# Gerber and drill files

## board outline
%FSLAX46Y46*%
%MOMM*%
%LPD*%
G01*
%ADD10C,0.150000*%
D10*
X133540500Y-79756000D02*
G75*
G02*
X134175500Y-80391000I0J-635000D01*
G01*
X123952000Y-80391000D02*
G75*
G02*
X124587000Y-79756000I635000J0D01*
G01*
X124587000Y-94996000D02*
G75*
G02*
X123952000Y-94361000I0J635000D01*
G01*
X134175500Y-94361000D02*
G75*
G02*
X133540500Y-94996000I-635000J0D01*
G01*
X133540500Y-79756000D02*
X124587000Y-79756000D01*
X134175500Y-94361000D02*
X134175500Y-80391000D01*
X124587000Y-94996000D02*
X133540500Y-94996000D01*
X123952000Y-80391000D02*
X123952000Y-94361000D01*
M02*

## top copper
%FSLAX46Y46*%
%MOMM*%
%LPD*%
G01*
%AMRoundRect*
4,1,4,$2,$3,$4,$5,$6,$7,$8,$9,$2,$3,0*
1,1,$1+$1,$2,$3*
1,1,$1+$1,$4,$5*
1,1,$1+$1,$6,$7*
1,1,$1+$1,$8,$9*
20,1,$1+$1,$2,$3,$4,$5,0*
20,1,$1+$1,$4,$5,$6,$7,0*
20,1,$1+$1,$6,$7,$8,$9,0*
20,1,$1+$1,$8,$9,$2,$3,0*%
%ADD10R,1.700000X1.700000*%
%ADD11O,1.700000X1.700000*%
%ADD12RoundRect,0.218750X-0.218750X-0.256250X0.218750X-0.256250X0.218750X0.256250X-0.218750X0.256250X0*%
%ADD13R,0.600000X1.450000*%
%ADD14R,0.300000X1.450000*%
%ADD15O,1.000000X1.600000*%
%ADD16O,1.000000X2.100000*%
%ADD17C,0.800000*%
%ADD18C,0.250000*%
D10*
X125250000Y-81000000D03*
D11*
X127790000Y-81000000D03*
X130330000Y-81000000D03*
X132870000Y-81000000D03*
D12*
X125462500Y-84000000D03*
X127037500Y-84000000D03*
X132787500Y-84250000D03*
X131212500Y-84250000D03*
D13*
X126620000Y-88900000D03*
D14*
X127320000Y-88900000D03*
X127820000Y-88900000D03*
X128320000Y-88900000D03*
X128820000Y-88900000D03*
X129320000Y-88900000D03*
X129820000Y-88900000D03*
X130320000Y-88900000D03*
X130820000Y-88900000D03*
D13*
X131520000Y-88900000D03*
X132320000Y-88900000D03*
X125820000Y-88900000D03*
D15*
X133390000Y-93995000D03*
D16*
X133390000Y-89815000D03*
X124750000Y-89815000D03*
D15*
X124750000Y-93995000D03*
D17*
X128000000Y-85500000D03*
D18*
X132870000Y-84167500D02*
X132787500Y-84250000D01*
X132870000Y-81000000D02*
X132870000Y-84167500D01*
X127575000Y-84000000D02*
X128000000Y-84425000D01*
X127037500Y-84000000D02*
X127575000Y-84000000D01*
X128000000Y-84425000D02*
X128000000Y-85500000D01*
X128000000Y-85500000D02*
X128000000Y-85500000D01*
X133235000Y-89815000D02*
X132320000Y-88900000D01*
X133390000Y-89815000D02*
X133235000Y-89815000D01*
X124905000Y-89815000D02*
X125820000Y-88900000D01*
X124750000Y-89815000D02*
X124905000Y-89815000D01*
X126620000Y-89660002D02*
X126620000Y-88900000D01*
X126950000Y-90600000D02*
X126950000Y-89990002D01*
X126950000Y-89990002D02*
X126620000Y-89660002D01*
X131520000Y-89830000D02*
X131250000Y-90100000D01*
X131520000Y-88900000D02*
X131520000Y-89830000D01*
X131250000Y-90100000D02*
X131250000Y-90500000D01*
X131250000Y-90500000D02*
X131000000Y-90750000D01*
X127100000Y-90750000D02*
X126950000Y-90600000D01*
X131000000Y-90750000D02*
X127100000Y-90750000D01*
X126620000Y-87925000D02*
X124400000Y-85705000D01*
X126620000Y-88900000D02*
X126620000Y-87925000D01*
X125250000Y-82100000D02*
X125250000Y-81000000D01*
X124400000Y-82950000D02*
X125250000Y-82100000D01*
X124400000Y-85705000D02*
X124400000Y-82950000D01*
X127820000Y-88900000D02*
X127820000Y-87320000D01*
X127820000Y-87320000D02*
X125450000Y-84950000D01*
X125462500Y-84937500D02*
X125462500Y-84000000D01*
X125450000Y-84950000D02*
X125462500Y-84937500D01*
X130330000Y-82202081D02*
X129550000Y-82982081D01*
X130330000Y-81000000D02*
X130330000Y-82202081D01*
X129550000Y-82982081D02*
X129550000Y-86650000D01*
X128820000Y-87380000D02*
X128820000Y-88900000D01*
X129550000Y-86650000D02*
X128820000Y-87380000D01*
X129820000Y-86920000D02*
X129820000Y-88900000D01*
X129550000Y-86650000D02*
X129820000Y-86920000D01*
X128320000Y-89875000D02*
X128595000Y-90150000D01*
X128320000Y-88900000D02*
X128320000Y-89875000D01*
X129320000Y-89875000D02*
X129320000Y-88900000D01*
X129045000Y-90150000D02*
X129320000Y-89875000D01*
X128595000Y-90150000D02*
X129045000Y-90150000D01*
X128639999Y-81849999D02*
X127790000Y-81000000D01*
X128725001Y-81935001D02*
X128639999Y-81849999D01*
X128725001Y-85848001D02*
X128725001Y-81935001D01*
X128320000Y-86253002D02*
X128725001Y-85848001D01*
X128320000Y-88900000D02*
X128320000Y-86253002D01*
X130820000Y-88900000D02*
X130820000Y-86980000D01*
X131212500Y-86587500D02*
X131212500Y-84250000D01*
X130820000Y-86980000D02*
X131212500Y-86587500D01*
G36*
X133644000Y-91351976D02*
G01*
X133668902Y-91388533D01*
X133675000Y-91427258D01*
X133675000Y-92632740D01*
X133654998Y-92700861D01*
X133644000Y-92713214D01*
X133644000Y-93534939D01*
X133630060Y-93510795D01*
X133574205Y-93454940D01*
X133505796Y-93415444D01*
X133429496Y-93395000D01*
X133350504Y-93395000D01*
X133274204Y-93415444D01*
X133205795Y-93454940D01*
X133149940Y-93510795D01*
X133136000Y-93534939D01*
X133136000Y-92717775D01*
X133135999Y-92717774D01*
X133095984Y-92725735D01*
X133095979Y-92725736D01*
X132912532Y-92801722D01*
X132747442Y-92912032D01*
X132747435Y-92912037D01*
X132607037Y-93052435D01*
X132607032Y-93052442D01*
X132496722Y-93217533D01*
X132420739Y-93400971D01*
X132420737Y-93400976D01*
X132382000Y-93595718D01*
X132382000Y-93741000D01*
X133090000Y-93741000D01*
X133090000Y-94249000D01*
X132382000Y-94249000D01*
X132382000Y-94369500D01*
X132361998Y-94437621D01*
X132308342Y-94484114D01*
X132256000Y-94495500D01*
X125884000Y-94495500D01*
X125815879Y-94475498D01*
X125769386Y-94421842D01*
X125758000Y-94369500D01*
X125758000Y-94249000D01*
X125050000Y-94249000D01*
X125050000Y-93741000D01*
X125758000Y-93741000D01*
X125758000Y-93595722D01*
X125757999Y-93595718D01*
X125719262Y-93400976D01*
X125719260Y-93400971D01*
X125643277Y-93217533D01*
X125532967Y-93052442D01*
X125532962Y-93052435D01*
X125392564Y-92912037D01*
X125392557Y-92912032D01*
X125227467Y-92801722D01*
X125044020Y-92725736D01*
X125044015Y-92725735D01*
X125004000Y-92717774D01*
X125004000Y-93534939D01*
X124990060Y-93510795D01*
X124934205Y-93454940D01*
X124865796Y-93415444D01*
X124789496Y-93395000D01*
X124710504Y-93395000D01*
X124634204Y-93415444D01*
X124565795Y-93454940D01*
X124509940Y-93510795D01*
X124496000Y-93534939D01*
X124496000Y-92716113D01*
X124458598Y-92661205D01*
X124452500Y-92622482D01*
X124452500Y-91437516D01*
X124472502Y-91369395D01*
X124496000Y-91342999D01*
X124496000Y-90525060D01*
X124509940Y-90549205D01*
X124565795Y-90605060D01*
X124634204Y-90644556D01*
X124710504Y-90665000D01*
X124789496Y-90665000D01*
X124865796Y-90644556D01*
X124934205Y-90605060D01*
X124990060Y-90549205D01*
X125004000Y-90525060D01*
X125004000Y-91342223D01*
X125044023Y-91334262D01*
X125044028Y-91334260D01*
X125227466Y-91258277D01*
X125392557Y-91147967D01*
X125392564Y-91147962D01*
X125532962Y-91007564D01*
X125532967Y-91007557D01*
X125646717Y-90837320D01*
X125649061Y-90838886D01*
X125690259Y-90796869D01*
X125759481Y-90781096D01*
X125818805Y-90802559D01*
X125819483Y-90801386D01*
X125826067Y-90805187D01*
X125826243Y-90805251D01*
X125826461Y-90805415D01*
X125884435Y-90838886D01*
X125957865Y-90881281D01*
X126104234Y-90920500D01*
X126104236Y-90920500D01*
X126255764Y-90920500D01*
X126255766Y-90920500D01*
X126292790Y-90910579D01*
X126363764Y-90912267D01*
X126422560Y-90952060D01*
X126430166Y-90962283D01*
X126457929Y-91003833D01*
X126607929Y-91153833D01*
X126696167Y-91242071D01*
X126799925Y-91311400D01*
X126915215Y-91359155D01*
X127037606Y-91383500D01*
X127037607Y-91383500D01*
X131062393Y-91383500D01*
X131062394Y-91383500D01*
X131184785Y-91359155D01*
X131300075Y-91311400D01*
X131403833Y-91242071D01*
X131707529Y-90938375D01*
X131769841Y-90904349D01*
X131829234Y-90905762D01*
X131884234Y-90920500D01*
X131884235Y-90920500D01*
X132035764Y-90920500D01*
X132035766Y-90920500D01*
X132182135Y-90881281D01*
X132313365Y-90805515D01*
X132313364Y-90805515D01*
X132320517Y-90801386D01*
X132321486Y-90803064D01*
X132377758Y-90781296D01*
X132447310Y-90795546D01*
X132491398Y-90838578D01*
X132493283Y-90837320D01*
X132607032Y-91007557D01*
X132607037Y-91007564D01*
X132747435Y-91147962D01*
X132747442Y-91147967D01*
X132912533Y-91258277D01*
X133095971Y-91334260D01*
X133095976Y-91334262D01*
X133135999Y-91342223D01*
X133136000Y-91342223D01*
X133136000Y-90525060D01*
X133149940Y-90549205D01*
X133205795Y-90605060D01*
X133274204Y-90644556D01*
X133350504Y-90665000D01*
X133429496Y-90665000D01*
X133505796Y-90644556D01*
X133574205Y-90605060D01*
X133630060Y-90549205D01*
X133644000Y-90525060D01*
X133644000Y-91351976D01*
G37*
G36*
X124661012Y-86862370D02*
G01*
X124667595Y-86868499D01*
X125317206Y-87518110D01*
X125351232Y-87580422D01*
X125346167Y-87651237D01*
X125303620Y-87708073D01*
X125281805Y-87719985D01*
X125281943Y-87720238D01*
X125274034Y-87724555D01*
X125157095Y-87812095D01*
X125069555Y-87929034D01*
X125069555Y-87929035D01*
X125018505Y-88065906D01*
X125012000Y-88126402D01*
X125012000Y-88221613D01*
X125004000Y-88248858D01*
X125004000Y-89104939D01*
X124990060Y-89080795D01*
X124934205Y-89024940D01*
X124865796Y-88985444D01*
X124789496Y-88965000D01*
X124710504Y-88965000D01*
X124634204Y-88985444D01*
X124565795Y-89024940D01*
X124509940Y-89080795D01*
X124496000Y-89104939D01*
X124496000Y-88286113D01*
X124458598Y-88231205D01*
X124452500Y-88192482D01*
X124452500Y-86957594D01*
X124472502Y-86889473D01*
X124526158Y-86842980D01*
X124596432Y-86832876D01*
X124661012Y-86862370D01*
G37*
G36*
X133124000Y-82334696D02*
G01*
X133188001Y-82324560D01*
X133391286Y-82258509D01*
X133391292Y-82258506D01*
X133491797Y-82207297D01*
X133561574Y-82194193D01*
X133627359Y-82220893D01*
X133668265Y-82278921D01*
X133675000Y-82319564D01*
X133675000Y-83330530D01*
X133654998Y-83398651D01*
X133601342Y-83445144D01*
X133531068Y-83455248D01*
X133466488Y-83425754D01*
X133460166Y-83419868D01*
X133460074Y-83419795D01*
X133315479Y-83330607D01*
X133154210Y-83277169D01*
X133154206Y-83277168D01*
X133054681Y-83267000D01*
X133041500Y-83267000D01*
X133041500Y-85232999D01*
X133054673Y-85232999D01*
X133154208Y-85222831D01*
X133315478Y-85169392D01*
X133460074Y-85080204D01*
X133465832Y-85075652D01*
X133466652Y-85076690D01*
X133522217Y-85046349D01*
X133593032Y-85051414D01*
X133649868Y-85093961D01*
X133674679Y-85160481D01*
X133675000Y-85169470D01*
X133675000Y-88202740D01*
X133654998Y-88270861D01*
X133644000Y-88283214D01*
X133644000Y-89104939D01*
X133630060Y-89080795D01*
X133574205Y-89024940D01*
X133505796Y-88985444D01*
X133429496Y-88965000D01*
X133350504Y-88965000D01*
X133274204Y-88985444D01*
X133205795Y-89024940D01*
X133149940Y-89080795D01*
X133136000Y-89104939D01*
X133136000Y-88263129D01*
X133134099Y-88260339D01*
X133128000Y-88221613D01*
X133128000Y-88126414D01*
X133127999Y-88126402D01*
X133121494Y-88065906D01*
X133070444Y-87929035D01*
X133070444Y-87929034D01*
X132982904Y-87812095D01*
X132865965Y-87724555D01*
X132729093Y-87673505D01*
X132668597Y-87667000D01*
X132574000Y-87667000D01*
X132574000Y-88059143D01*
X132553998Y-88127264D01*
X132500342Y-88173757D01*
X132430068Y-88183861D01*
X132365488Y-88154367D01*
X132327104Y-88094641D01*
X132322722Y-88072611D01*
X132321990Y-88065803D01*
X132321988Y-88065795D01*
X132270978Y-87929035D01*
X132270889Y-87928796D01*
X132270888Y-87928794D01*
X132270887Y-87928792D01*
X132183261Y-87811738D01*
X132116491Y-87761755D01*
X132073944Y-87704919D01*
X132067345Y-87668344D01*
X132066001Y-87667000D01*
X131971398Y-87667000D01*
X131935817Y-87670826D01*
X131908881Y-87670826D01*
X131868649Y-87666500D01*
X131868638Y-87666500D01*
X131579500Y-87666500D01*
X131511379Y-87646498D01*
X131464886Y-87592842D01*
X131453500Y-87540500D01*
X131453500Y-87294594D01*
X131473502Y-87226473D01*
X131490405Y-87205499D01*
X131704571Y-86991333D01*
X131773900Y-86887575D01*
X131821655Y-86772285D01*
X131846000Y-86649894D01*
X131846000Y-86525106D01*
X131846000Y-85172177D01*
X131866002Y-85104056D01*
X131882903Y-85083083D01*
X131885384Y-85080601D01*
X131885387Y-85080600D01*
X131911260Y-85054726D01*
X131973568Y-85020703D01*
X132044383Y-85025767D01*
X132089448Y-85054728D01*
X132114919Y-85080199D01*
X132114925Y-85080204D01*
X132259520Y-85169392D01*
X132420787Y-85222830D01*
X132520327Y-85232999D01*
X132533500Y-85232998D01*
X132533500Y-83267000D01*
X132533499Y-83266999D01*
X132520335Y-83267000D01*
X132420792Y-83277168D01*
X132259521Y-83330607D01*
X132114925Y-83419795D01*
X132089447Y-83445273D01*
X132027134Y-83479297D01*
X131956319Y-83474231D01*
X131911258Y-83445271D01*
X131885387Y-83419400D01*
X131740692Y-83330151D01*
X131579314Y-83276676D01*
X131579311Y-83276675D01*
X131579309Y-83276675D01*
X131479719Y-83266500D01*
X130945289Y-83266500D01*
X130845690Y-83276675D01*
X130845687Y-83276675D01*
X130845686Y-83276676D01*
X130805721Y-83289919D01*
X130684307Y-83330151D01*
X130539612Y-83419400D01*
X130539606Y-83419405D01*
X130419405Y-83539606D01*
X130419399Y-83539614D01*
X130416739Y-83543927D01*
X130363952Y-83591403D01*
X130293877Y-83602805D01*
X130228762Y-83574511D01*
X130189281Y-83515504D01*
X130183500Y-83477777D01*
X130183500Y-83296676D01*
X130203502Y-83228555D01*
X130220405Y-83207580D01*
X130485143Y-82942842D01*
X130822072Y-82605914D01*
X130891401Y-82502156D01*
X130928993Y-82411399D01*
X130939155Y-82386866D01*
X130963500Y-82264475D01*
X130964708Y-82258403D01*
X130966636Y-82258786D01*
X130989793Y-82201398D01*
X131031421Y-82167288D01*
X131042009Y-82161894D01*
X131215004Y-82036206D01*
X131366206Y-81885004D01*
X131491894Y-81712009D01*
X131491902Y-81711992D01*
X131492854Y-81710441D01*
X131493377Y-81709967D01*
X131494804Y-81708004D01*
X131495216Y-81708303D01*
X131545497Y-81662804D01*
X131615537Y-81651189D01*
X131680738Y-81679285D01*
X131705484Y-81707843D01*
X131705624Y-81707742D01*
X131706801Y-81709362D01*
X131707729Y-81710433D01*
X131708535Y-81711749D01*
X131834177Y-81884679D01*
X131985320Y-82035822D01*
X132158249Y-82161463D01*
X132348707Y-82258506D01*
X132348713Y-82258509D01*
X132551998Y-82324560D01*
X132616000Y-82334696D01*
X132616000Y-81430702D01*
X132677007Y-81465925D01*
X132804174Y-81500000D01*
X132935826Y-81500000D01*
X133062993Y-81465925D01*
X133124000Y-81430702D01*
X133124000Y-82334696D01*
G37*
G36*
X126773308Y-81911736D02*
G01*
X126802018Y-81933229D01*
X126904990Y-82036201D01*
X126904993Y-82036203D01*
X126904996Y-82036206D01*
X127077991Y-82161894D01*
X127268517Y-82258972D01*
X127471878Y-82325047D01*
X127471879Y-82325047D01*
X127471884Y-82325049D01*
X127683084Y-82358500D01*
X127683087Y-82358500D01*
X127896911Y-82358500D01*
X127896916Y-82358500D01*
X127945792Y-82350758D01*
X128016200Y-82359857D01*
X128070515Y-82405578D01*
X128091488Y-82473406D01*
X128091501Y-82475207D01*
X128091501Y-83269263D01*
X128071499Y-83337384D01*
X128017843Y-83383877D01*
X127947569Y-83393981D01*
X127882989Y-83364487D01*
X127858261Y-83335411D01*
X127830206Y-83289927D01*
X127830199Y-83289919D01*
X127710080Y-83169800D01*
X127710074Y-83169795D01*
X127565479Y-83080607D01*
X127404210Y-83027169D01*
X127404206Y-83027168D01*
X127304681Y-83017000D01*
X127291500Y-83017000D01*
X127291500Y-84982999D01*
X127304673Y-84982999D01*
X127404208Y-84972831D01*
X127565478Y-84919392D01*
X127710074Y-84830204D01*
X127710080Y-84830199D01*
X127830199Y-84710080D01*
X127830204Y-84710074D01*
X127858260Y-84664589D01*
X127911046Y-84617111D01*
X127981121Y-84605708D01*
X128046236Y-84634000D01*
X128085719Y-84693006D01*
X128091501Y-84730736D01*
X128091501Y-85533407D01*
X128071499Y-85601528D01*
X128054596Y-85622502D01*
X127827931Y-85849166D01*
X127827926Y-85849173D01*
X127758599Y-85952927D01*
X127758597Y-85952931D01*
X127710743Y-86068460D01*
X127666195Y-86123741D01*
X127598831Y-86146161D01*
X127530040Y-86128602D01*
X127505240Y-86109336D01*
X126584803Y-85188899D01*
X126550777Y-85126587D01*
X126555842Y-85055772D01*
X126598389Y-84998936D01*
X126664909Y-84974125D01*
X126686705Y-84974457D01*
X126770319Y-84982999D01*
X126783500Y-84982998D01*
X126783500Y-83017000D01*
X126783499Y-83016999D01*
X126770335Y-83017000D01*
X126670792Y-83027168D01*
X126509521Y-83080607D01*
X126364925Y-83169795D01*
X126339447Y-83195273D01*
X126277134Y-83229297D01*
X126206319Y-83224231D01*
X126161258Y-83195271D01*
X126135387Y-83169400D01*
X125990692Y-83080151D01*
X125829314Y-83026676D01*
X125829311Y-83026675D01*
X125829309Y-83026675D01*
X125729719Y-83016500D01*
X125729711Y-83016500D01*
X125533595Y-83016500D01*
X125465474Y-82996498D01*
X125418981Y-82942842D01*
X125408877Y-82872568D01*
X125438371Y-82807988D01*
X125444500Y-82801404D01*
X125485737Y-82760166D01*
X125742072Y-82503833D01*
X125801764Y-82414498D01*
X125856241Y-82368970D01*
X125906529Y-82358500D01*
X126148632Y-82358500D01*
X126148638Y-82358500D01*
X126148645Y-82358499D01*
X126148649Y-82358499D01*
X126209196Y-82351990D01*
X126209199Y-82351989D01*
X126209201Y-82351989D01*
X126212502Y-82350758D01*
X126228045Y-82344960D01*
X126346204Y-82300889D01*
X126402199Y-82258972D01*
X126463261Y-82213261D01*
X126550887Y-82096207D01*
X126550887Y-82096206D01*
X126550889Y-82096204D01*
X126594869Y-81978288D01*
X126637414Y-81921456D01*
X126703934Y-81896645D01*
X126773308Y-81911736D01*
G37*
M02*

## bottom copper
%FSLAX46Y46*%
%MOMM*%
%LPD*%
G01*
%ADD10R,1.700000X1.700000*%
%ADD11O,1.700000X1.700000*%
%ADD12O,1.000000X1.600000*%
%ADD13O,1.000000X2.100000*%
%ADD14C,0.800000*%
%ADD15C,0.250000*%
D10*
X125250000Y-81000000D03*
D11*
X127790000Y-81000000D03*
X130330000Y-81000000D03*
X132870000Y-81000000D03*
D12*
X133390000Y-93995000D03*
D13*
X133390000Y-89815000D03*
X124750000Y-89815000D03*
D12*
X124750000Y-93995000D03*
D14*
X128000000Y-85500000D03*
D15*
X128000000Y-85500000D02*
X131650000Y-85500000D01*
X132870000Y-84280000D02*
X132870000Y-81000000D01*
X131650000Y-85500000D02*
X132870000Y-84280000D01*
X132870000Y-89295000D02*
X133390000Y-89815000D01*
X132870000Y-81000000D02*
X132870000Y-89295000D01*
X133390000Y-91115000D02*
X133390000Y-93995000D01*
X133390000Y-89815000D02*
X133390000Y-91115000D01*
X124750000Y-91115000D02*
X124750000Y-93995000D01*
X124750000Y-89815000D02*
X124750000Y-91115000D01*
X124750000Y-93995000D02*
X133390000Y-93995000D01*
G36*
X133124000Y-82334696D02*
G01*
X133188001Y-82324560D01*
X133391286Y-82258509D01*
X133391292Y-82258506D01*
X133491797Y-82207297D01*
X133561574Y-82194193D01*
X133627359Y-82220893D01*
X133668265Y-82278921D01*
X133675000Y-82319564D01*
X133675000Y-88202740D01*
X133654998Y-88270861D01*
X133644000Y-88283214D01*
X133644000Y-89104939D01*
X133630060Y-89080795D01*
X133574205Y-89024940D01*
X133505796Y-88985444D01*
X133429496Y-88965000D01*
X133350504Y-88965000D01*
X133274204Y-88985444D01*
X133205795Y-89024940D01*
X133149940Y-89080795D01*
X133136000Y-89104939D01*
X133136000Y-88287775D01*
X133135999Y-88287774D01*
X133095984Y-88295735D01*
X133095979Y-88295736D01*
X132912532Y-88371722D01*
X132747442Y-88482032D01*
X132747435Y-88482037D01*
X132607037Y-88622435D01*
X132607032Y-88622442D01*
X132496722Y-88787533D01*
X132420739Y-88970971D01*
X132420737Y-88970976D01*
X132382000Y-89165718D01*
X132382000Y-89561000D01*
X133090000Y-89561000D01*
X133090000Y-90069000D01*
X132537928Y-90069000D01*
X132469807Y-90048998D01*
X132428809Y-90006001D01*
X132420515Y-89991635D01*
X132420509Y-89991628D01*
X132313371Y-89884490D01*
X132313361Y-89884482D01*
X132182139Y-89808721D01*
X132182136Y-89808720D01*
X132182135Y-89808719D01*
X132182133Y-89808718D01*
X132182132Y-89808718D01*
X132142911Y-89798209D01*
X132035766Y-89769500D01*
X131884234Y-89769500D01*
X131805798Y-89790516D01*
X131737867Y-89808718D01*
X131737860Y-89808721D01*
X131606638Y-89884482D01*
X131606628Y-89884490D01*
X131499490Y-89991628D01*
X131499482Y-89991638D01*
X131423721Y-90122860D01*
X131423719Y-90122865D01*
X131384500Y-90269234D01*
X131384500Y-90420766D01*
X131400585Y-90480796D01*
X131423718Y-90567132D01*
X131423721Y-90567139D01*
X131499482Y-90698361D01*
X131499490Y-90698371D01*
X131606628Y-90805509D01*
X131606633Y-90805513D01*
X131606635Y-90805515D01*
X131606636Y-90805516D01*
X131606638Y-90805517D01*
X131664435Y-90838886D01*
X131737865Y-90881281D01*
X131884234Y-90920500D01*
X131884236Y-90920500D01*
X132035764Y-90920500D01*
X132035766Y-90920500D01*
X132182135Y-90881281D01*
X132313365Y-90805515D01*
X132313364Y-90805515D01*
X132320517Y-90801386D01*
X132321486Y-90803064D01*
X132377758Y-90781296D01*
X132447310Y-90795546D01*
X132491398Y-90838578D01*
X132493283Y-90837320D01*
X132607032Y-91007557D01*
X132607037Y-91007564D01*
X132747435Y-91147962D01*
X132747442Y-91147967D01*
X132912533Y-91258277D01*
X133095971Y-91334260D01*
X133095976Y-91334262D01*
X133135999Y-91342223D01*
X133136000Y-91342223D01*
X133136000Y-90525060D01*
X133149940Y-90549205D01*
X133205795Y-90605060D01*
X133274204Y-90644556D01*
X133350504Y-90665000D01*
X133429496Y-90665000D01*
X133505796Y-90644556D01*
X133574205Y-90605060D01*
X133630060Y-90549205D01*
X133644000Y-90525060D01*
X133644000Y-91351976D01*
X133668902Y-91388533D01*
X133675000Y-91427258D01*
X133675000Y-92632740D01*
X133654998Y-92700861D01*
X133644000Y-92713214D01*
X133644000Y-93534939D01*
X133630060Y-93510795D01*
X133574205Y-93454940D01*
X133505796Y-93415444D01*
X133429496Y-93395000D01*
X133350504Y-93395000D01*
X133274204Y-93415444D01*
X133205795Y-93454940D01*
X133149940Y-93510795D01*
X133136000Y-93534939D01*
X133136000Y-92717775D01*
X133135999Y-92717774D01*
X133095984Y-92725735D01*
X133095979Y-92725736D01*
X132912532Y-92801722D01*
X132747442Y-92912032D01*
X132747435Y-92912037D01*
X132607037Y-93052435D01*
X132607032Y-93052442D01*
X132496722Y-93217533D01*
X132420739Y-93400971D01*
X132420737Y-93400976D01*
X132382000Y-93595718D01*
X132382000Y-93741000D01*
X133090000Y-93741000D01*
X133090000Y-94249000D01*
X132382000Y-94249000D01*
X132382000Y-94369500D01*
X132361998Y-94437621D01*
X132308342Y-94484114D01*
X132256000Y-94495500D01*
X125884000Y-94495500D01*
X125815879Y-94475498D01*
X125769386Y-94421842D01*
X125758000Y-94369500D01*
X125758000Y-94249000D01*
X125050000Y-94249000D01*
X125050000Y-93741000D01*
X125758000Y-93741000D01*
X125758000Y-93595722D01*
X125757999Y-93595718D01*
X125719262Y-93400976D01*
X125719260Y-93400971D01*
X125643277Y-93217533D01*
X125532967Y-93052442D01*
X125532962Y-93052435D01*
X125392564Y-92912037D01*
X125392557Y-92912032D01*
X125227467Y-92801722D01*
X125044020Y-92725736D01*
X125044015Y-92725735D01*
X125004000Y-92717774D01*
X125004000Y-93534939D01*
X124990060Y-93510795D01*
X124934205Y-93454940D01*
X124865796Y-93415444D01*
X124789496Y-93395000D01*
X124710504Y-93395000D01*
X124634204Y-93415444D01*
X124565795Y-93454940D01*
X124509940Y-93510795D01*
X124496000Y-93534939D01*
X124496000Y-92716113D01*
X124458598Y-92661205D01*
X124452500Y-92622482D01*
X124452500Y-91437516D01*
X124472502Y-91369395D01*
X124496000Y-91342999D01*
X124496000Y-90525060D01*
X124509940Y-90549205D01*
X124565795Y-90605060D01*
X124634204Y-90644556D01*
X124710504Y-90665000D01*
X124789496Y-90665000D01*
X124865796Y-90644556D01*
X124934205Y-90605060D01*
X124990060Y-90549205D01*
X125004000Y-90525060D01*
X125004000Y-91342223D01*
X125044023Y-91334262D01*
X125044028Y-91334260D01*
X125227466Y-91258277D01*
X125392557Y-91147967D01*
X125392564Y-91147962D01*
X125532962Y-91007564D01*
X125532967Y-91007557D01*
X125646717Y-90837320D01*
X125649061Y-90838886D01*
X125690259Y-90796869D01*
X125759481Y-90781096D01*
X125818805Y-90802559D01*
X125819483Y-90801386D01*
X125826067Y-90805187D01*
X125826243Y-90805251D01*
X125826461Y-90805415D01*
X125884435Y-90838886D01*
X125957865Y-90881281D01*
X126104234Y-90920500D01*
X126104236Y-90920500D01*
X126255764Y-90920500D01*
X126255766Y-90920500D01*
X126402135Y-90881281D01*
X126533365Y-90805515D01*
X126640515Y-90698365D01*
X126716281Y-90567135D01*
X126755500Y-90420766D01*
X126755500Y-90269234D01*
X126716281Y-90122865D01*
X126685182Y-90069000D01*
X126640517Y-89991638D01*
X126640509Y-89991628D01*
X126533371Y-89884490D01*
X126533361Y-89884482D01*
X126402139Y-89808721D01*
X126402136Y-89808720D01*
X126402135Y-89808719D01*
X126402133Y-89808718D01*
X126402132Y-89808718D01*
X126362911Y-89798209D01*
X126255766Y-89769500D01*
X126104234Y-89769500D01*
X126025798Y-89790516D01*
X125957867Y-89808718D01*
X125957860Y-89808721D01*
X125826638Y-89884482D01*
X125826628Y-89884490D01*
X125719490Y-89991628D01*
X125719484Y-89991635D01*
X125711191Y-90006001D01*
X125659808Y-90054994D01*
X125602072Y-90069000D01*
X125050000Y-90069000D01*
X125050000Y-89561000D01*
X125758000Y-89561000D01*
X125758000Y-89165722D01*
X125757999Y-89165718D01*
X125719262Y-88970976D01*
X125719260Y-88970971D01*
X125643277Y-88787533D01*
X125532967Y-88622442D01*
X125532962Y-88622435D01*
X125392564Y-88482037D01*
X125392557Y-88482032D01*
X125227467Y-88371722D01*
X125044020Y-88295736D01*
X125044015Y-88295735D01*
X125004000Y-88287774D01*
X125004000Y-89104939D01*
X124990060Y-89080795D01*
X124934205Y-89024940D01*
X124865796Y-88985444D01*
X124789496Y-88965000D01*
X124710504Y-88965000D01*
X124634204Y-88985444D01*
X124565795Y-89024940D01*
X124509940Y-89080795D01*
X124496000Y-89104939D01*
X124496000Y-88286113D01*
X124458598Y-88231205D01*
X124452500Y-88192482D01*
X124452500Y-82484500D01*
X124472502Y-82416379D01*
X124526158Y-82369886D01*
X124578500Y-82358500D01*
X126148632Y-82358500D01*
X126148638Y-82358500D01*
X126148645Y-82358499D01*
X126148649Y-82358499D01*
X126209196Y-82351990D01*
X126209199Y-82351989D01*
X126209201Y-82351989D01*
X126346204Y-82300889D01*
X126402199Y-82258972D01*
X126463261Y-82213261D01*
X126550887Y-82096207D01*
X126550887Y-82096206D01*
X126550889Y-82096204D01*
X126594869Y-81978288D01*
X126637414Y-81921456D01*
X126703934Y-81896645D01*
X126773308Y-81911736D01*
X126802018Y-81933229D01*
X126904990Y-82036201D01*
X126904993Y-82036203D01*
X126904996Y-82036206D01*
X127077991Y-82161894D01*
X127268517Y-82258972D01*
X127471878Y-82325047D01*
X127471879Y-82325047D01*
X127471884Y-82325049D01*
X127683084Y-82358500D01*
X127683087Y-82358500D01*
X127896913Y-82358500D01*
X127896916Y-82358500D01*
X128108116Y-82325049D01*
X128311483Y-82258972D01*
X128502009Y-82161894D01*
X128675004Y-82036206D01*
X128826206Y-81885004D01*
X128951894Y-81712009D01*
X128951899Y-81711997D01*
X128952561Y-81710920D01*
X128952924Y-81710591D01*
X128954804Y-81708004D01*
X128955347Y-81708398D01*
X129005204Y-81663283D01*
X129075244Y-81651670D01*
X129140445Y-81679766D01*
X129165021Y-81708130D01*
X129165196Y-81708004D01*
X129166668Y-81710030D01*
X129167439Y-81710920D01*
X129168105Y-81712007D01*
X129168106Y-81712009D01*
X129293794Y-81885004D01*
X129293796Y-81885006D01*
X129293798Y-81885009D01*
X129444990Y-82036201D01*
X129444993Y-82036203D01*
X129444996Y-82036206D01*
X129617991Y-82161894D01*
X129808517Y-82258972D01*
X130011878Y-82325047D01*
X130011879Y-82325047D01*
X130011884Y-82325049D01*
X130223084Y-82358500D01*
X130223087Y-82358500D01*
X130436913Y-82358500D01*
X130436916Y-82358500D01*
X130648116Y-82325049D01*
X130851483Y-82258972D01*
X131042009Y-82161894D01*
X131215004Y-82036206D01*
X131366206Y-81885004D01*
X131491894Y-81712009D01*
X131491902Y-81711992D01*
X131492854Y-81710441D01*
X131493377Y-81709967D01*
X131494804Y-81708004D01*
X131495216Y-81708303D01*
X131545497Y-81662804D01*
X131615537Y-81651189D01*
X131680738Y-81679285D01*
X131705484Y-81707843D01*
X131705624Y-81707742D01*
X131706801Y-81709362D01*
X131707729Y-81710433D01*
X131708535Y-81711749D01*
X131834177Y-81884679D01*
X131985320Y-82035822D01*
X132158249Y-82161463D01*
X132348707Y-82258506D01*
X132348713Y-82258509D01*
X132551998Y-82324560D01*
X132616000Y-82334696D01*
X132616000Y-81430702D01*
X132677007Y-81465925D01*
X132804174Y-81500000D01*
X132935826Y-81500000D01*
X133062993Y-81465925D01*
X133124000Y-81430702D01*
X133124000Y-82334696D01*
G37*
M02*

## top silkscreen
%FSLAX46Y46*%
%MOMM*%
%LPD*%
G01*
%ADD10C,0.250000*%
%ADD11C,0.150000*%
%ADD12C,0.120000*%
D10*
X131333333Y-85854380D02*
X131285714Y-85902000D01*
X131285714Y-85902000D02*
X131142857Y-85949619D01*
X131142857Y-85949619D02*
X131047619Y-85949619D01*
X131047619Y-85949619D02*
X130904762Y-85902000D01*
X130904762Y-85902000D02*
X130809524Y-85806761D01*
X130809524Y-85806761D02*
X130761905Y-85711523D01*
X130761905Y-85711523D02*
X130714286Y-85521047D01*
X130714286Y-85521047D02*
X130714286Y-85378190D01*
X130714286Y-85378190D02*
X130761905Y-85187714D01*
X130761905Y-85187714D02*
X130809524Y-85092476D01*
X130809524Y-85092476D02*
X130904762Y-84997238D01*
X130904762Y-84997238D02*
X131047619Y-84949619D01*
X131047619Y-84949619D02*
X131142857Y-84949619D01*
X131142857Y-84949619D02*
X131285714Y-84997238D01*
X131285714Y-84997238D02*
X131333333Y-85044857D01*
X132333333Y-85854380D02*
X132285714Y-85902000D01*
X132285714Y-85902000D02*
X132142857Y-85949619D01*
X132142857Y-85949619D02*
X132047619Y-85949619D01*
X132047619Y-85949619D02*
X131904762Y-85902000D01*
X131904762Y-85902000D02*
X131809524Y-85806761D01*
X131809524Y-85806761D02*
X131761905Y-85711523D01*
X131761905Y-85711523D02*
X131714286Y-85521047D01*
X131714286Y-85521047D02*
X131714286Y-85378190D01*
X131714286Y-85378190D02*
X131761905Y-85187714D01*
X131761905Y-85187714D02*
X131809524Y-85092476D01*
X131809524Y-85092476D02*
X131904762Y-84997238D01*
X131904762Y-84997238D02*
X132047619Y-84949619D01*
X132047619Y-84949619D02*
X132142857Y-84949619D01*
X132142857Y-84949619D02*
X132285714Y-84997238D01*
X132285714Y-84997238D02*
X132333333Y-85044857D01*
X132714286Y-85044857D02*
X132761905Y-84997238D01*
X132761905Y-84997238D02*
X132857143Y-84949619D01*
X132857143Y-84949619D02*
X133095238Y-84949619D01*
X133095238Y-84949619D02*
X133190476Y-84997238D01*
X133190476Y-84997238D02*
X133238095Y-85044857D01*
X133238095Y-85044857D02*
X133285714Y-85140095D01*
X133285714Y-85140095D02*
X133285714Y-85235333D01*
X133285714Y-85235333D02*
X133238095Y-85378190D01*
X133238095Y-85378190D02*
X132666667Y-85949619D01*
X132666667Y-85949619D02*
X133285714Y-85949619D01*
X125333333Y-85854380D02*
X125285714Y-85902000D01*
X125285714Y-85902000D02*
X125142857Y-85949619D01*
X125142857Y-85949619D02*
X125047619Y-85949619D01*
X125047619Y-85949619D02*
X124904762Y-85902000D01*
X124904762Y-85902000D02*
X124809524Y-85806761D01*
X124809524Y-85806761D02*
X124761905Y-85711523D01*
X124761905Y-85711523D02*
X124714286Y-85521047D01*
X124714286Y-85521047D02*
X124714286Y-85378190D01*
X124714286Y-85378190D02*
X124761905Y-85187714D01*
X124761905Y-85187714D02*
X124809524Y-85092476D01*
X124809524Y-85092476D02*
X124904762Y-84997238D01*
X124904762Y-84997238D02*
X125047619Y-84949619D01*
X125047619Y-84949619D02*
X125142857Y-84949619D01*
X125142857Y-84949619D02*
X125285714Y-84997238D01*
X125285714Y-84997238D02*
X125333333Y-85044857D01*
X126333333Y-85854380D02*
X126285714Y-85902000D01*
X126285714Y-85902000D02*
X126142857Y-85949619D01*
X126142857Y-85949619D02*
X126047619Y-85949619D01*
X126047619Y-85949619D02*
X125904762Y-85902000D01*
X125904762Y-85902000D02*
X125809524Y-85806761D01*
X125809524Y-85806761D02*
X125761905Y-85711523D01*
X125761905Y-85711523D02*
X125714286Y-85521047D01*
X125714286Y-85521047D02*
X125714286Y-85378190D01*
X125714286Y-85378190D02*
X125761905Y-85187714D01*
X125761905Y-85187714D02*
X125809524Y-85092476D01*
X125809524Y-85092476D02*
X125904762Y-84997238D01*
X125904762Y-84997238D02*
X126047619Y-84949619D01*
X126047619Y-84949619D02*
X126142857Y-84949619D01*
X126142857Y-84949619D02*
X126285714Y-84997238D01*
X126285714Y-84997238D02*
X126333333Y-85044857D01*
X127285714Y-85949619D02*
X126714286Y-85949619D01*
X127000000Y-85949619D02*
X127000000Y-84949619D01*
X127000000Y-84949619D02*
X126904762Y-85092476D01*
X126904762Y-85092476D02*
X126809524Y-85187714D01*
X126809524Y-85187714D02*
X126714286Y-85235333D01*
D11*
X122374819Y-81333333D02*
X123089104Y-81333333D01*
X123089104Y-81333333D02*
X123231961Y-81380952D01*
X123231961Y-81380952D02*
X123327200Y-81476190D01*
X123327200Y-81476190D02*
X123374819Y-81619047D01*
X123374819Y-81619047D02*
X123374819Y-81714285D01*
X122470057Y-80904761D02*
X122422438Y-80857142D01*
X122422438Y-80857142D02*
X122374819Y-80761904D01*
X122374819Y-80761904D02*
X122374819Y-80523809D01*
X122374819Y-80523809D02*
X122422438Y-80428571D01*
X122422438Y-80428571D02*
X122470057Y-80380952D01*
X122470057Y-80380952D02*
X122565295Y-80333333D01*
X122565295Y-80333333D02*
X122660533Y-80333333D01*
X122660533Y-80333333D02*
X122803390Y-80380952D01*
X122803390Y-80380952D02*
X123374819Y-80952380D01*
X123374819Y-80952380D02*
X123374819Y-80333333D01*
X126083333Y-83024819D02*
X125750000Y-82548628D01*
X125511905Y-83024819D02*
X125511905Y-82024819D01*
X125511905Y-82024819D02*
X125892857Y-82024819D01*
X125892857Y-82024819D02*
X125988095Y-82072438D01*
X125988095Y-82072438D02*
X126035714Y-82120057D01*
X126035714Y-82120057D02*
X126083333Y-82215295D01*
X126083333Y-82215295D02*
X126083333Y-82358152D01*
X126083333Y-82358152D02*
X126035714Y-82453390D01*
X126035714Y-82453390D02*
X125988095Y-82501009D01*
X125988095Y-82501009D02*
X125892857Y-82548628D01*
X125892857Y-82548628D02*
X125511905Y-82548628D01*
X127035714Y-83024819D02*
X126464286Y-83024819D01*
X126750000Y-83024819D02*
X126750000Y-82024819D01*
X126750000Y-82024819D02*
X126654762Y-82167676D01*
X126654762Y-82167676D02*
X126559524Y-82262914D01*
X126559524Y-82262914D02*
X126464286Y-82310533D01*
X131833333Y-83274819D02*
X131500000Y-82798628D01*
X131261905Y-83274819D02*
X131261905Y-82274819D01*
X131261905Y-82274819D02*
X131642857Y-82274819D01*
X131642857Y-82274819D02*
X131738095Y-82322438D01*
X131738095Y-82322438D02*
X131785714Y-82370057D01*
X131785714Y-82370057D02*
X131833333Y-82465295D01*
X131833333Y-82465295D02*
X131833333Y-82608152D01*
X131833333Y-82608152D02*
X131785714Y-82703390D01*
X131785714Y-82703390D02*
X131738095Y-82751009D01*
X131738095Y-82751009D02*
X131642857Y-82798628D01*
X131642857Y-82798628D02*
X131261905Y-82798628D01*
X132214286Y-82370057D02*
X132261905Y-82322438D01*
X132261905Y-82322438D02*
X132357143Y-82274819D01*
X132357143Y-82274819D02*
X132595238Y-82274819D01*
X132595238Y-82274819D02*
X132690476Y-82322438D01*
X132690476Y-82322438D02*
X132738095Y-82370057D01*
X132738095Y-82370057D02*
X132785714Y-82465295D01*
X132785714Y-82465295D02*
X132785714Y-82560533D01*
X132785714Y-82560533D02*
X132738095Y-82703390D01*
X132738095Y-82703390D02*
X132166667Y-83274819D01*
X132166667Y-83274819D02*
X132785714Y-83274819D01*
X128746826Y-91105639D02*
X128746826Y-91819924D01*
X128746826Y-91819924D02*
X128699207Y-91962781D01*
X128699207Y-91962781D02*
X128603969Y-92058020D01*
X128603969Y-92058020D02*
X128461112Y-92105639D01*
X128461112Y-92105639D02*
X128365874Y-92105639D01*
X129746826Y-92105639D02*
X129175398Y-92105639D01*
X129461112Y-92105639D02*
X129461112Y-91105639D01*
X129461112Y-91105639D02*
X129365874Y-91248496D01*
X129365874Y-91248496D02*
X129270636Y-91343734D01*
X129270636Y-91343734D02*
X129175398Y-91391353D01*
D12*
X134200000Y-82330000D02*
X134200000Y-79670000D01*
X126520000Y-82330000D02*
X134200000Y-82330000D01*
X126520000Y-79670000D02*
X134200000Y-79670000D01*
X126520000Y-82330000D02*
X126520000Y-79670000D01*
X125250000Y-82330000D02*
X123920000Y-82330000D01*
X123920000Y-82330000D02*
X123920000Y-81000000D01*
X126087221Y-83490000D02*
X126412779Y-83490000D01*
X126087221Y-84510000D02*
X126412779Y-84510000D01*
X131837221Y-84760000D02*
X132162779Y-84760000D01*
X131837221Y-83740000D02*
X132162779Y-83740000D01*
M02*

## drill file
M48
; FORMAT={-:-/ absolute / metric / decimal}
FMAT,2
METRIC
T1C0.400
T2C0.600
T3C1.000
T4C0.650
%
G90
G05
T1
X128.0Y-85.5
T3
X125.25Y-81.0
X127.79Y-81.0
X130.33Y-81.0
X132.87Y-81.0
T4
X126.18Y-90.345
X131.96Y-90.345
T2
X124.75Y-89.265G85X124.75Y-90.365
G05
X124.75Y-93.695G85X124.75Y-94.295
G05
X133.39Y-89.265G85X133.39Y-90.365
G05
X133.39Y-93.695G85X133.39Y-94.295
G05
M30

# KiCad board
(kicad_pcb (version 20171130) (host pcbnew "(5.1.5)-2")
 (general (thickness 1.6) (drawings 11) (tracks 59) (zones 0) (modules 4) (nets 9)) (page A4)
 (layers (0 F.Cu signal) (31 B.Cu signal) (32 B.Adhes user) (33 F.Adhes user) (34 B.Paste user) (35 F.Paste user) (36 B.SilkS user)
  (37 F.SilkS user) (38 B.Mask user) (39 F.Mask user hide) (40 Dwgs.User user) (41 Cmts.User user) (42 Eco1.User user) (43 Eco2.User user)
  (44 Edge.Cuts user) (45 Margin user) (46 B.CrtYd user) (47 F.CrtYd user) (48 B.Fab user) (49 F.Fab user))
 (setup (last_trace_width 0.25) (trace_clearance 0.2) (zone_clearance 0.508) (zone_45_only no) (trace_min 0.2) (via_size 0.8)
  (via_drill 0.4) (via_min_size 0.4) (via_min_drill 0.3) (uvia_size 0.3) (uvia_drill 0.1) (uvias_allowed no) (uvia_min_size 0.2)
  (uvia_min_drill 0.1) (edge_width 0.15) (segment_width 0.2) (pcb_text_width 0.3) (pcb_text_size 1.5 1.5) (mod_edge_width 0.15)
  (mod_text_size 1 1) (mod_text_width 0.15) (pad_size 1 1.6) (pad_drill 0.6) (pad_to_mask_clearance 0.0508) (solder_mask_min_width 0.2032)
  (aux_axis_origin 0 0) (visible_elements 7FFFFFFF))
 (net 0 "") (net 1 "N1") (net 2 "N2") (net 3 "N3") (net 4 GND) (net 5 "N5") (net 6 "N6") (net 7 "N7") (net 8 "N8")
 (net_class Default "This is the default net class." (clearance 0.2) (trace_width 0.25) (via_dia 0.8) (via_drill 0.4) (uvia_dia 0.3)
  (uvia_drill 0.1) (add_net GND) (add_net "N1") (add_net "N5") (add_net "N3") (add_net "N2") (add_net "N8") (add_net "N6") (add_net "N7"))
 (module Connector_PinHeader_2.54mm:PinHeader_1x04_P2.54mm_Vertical (layer F.Cu) (at 125.25 81 90)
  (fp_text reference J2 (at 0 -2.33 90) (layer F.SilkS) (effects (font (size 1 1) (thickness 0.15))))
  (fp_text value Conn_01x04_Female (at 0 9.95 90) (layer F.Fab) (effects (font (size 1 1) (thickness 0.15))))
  (fp_line (start -1.33 8.95) (end 1.33 8.95) (layer F.SilkS) (width 0.12))
  (fp_line (start -1.33 1.27) (end -1.33 8.95) (layer F.SilkS) (width 0.12))
  (fp_line (start 1.33 1.27) (end 1.33 8.95) (layer F.SilkS) (width 0.12))
  (fp_line (start -1.33 1.27) (end 1.33 1.27) (layer F.SilkS) (width 0.12))
  (fp_line (start -1.33 0) (end -1.33 -1.33) (layer F.SilkS) (width 0.12))
  (fp_line (start -1.33 -1.33) (end 0 -1.33) (layer F.SilkS) (width 0.12))
  (pad 1 thru_hole rect (at 0 0 90) (size 1.7 1.7) (drill 1) (layers *.Cu *.Mask) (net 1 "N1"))
  (pad 2 thru_hole oval (at 0 2.54 90) (size 1.7 1.7) (drill 1) (layers *.Cu *.Mask) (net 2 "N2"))
  (pad 3 thru_hole oval (at 0 5.08 90) (size 1.7 1.7) (drill 1) (layers *.Cu *.Mask) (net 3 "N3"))
  (pad 4 thru_hole oval (at 0 7.62 90) (size 1.7 1.7) (drill 1) (layers *.Cu *.Mask) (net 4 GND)))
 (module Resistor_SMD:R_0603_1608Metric (layer F.Cu) (at 126.25 84)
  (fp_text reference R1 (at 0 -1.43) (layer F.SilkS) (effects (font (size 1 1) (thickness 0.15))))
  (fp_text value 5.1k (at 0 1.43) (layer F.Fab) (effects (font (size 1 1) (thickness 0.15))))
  (fp_line (start -0.162779 -0.51) (end 0.162779 -0.51) (layer F.SilkS) (width 0.12))
  (fp_line (start -0.162779 0.51) (end 0.162779 0.51) (layer F.SilkS) (width 0.12))
  (pad 1 smd roundrect (at -0.7875 0) (size 0.875 0.95) (layers F.Cu F.Paste F.Mask) (roundrect_rratio 0.25) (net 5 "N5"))
  (pad 2 smd roundrect (at 0.7875 0) (size 0.875 0.95) (layers F.Cu F.Paste F.Mask) (roundrect_rratio 0.25) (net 4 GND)))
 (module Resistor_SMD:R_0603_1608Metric (layer F.Cu) (at 132 84.25)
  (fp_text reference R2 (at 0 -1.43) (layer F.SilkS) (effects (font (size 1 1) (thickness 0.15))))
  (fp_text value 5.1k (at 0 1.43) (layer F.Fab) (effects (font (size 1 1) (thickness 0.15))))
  (fp_line (start -0.162779 0.51) (end 0.162779 0.51) (layer F.SilkS) (width 0.12))
  (fp_line (start -0.162779 -0.51) (end 0.162779 -0.51) (layer F.SilkS) (width 0.12))
  (pad 2 smd roundrect (at 0.7875 0) (size 0.875 0.95) (layers F.Cu F.Paste F.Mask) (roundrect_rratio 0.25) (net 4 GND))
  (pad 1 smd roundrect (at -0.7875 0) (size 0.875 0.95) (layers F.Cu F.Paste F.Mask) (roundrect_rratio 0.25) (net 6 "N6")))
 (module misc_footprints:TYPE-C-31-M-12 (layer F.Cu) (at 129.07 88.9)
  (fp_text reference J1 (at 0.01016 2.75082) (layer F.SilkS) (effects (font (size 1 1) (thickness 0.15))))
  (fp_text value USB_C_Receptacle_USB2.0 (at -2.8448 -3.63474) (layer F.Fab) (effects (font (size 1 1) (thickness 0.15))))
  (pad A4|B9 smd rect (at -2.45 0) (size 0.6 1.45) (layers F.Cu F.Paste F.Mask) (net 1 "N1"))
  (pad B8 smd rect (at -1.75 0) (size 0.3 1.45) (layers F.Cu F.Paste F.Mask) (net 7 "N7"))
  (pad A5 smd rect (at -1.25 0) (size 0.3 1.45) (layers F.Cu F.Paste F.Mask) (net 5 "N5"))
  (pad B7 smd rect (at -0.75 0) (size 0.3 1.45) (layers F.Cu F.Paste F.Mask) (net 2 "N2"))
  (pad A6 smd rect (at -0.25 0) (size 0.3 1.45) (layers F.Cu F.Paste F.Mask) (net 3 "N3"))
  (pad A7 smd rect (at 0.25 0) (size 0.3 1.45) (layers F.Cu F.Paste F.Mask) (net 2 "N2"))
  (pad B6 smd rect (at 0.75 0) (size 0.3 1.45) (layers F.Cu F.Paste F.Mask) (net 3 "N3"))
  (pad A8 smd rect (at 1.25 0) (size 0.3 1.45) (layers F.Cu F.Paste F.Mask) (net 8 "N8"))
  (pad B5 smd rect (at 1.75 0) (size 0.3 1.45) (layers F.Cu F.Paste F.Mask) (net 6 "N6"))
  (pad B4|A9 smd rect (at 2.45 0) (size 0.6 1.45) (layers F.Cu F.Paste F.Mask) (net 1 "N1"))
  (pad B1|A12 smd rect (at 3.25 0) (size 0.6 1.45) (layers F.Cu F.Paste F.Mask) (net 4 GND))
  (pad A1|B12 smd rect (at -3.25 0) (size 0.6 1.45) (layers F.Cu F.Paste F.Mask) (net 4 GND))
  (pad GND thru_hole oval (at 4.32 5.095) (size 1 1.6) (drill oval 0.6 1.2) (layers *.Cu *.Mask) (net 4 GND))
  (pad GND thru_hole oval (at 4.32 0.915) (size 1 2.1) (drill oval 0.6 1.7) (layers *.Cu *.Mask) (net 4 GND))
  (pad GND thru_hole oval (at -4.32 0.915) (size 1 2.1) (drill oval 0.6 1.7) (layers *.Cu *.Mask) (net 4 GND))
  (pad GND thru_hole oval (at -4.32 5.095) (size 1 1.6) (drill oval 0.6 1.2) (layers *.Cu *.Mask) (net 4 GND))
  (pad "" np_thru_hole circle (at 2.89 1.445) (size 0.65 0.65) (drill 0.65) (layers *.Cu *.Mask))
  (pad "" np_thru_hole circle (at -2.89 1.445) (size 0.65 0.65) (drill 0.65) (layers *.Cu *.Mask)))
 (gr_arc (start 133.5405 80.391) (end 134.1755 80.391) (angle -90) (layer Edge.Cuts) (width 0.15))
 (gr_arc (start 124.587 80.391) (end 124.587 79.756) (angle -90) (layer Edge.Cuts) (width 0.15))
 (gr_arc (start 124.587 94.361) (end 123.952 94.361) (angle -90) (layer Edge.Cuts) (width 0.15))
 (gr_arc (start 133.5405 94.361) (end 133.5405 94.996) (angle -90) (layer Edge.Cuts) (width 0.15))
 (gr_line (start 133.5405 79.756) (end 124.587 79.756) (layer Edge.Cuts) (width 0.15))
 (gr_line (start 134.1755 94.361) (end 134.1755 80.391) (layer Edge.Cuts) (width 0.15))
 (gr_line (start 124.587 94.996) (end 133.5405 94.996) (layer Edge.Cuts) (width 0.15))
 (gr_line (start 123.952 80.391) (end 123.952 94.361) (layer Edge.Cuts) (width 0.15))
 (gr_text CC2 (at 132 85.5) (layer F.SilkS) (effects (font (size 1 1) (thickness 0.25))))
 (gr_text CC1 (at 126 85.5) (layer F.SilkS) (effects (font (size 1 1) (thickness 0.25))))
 (segment (start 132.87 84.1675) (end 132.7875 84.25) (width 0.25) (layer F.Cu) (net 4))
 (segment (start 132.87 81) (end 132.87 84.1675) (width 0.25) (layer F.Cu) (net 4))
 (segment (start 127.575 84) (end 128 84.425) (width 0.25) (layer F.Cu) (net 4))
 (segment (start 127.0375 84) (end 127.575 84) (width 0.25) (layer F.Cu) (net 4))
 (segment (start 128 84.425) (end 128 85.5) (width 0.25) (layer F.Cu) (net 4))
 (segment (start 128 85.5) (end 128 85.5) (width 0.25) (layer F.Cu) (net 4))
 (via (at 128 85.5) (size 0.8) (drill 0.4) (layers F.Cu B.Cu) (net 4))
 (segment (start 128 85.5) (end 131.65 85.5) (width 0.25) (layer B.Cu) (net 4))
 (segment (start 132.87 84.28) (end 132.87 81) (width 0.25) (layer B.Cu) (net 4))
 (segment (start 131.65 85.5) (end 132.87 84.28) (width 0.25) (layer B.Cu) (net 4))
 (segment (start 132.87 89.295) (end 133.39 89.815) (width 0.25) (layer B.Cu) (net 4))
 (segment (start 132.87 81) (end 132.87 89.295) (width 0.25) (layer B.Cu) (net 4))
 (segment (start 133.39 91.115) (end 133.39 93.995) (width 0.25) (layer B.Cu) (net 4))
 (segment (start 133.39 89.815) (end 133.39 91.115) (width 0.25) (layer B.Cu) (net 4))
 (segment (start 124.75 91.115) (end 124.75 93.995) (width 0.25) (layer B.Cu) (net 4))
 (segment (start 124.75 89.815) (end 124.75 91.115) (width 0.25) (layer B.Cu) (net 4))
 (segment (start 124.75 93.995) (end 133.39 93.995) (width 0.25) (layer B.Cu) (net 4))
 (segment (start 133.235 89.815) (end 132.32 88.9) (width 0.25) (layer F.Cu) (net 4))
 (segment (start 133.39 89.815) (end 133.235 89.815) (width 0.25) (layer F.Cu) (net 4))
 (segment (start 124.905 89.815) (end 125.82 88.9) (width 0.25) (layer F.Cu) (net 4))
 (segment (start 124.75 89.815) (end 124.905 89.815) (width 0.25) (layer F.Cu) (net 4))
 (segment (start 126.62 89.660002) (end 126.62 88.9) (width 0.25) (layer F.Cu) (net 1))
 (segment (start 126.95 90.6) (end 126.95 89.990002) (width 0.25) (layer F.Cu) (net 1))
 (segment (start 126.95 89.990002) (end 126.62 89.660002) (width 0.25) (layer F.Cu) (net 1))
 (segment (start 131.52 89.83) (end 131.25 90.1) (width 0.25) (layer F.Cu) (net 1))
 (segment (start 131.52 88.9) (end 131.52 89.83) (width 0.25) (layer F.Cu) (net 1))
 (segment (start 131.25 90.1) (end 131.25 90.5) (width 0.25) (layer F.Cu) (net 1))
 (segment (start 131.25 90.5) (end 131 90.75) (width 0.25) (layer F.Cu) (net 1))
 (segment (start 127.1 90.75) (end 126.95 90.6) (width 0.25) (layer F.Cu) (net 1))
 (segment (start 131 90.75) (end 127.1 90.75) (width 0.25) (layer F.Cu) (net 1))
 (segment (start 126.62 87.925) (end 124.4 85.705) (width 0.25) (layer F.Cu) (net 1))
 (segment (start 126.62 88.9) (end 126.62 87.925) (width 0.25) (layer F.Cu) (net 1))
 (segment (start 125.25 82.1) (end 125.25 81) (width 0.25) (layer F.Cu) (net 1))
 (segment (start 124.4 82.95) (end 125.25 82.1) (width 0.25) (layer F.Cu) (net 1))
 (segment (start 124.4 85.705) (end 124.4 82.95) (width 0.25) (layer F.Cu) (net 1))
 (segment (start 127.82 88.9) (end 127.82 87.32) (width 0.25) (layer F.Cu) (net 5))
 (segment (start 127.82 87.32) (end 125.45 84.95) (width 0.25) (layer F.Cu) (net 5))
 (segment (start 125.4625 84.9375) (end 125.4625 84) (width 0.25) (layer F.Cu) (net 5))
 (segment (start 125.45 84.95) (end 125.4625 84.9375) (width 0.25) (layer F.Cu) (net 5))
 (segment (start 130.33 82.202081) (end 129.55 82.982081) (width 0.25) (layer F.Cu) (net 3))
 (segment (start 130.33 81) (end 130.33 82.202081) (width 0.25) (layer F.Cu) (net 3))
 (segment (start 129.55 82.982081) (end 129.55 86.65) (width 0.25) (layer F.Cu) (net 3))
 (segment (start 128.82 87.38) (end 128.82 88.9) (width 0.25) (layer F.Cu) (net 3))
 (segment (start 129.55 86.65) (end 128.82 87.38) (width 0.25) (layer F.Cu) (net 3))
 (segment (start 129.82 86.92) (end 129.82 88.9) (width 0.25) (layer F.Cu) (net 3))
 (segment (start 129.55 86.65) (end 129.82 86.92) (width 0.25) (layer F.Cu) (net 3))
 (segment (start 128.32 89.875) (end 128.595 90.15) (width 0.25) (layer F.Cu) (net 2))
 (segment (start 128.32 88.9) (end 128.32 89.875) (width 0.25) (layer F.Cu) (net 2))
 (segment (start 129.32 89.875) (end 129.32 88.9) (width 0.25) (layer F.Cu) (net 2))
 (segment (start 129.045 90.15) (end 129.32 89.875) (width 0.25) (layer F.Cu) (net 2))
 (segment (start 128.595 90.15) (end 129.045 90.15) (width 0.25) (layer F.Cu) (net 2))
 (segment (start 128.639999 81.849999) (end 127.79 81) (width 0.25) (layer F.Cu) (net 2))
 (segment (start 128.725001 81.935001) (end 128.639999 81.849999) (width 0.25) (layer F.Cu) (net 2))
 (segment (start 128.725001 85.848001) (end 128.725001 81.935001) (width 0.25) (layer F.Cu) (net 2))
 (segment (start 128.32 86.253002) (end 128.725001 85.848001) (width 0.25) (layer F.Cu) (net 2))
 (segment (start 128.32 88.9) (end 128.32 86.253002) (width 0.25) (layer F.Cu) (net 2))
 (segment (start 130.82 88.9) (end 130.82 86.98) (width 0.25) (layer F.Cu) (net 6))
 (segment (start 131.2125 86.5875) (end 131.2125 84.25) (width 0.25) (layer F.Cu) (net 6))
 (segment (start 130.82 86.98) (end 131.2125 86.5875) (width 0.25) (layer F.Cu) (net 6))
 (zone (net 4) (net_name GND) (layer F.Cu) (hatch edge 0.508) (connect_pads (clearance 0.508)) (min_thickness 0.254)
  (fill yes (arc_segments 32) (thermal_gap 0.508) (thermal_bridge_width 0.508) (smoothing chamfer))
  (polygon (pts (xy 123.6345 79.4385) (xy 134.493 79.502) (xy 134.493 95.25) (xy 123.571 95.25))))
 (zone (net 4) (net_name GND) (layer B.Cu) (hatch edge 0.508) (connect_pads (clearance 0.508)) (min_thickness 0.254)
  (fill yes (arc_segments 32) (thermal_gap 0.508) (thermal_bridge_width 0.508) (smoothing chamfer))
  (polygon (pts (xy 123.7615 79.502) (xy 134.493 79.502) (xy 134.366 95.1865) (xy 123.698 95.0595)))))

